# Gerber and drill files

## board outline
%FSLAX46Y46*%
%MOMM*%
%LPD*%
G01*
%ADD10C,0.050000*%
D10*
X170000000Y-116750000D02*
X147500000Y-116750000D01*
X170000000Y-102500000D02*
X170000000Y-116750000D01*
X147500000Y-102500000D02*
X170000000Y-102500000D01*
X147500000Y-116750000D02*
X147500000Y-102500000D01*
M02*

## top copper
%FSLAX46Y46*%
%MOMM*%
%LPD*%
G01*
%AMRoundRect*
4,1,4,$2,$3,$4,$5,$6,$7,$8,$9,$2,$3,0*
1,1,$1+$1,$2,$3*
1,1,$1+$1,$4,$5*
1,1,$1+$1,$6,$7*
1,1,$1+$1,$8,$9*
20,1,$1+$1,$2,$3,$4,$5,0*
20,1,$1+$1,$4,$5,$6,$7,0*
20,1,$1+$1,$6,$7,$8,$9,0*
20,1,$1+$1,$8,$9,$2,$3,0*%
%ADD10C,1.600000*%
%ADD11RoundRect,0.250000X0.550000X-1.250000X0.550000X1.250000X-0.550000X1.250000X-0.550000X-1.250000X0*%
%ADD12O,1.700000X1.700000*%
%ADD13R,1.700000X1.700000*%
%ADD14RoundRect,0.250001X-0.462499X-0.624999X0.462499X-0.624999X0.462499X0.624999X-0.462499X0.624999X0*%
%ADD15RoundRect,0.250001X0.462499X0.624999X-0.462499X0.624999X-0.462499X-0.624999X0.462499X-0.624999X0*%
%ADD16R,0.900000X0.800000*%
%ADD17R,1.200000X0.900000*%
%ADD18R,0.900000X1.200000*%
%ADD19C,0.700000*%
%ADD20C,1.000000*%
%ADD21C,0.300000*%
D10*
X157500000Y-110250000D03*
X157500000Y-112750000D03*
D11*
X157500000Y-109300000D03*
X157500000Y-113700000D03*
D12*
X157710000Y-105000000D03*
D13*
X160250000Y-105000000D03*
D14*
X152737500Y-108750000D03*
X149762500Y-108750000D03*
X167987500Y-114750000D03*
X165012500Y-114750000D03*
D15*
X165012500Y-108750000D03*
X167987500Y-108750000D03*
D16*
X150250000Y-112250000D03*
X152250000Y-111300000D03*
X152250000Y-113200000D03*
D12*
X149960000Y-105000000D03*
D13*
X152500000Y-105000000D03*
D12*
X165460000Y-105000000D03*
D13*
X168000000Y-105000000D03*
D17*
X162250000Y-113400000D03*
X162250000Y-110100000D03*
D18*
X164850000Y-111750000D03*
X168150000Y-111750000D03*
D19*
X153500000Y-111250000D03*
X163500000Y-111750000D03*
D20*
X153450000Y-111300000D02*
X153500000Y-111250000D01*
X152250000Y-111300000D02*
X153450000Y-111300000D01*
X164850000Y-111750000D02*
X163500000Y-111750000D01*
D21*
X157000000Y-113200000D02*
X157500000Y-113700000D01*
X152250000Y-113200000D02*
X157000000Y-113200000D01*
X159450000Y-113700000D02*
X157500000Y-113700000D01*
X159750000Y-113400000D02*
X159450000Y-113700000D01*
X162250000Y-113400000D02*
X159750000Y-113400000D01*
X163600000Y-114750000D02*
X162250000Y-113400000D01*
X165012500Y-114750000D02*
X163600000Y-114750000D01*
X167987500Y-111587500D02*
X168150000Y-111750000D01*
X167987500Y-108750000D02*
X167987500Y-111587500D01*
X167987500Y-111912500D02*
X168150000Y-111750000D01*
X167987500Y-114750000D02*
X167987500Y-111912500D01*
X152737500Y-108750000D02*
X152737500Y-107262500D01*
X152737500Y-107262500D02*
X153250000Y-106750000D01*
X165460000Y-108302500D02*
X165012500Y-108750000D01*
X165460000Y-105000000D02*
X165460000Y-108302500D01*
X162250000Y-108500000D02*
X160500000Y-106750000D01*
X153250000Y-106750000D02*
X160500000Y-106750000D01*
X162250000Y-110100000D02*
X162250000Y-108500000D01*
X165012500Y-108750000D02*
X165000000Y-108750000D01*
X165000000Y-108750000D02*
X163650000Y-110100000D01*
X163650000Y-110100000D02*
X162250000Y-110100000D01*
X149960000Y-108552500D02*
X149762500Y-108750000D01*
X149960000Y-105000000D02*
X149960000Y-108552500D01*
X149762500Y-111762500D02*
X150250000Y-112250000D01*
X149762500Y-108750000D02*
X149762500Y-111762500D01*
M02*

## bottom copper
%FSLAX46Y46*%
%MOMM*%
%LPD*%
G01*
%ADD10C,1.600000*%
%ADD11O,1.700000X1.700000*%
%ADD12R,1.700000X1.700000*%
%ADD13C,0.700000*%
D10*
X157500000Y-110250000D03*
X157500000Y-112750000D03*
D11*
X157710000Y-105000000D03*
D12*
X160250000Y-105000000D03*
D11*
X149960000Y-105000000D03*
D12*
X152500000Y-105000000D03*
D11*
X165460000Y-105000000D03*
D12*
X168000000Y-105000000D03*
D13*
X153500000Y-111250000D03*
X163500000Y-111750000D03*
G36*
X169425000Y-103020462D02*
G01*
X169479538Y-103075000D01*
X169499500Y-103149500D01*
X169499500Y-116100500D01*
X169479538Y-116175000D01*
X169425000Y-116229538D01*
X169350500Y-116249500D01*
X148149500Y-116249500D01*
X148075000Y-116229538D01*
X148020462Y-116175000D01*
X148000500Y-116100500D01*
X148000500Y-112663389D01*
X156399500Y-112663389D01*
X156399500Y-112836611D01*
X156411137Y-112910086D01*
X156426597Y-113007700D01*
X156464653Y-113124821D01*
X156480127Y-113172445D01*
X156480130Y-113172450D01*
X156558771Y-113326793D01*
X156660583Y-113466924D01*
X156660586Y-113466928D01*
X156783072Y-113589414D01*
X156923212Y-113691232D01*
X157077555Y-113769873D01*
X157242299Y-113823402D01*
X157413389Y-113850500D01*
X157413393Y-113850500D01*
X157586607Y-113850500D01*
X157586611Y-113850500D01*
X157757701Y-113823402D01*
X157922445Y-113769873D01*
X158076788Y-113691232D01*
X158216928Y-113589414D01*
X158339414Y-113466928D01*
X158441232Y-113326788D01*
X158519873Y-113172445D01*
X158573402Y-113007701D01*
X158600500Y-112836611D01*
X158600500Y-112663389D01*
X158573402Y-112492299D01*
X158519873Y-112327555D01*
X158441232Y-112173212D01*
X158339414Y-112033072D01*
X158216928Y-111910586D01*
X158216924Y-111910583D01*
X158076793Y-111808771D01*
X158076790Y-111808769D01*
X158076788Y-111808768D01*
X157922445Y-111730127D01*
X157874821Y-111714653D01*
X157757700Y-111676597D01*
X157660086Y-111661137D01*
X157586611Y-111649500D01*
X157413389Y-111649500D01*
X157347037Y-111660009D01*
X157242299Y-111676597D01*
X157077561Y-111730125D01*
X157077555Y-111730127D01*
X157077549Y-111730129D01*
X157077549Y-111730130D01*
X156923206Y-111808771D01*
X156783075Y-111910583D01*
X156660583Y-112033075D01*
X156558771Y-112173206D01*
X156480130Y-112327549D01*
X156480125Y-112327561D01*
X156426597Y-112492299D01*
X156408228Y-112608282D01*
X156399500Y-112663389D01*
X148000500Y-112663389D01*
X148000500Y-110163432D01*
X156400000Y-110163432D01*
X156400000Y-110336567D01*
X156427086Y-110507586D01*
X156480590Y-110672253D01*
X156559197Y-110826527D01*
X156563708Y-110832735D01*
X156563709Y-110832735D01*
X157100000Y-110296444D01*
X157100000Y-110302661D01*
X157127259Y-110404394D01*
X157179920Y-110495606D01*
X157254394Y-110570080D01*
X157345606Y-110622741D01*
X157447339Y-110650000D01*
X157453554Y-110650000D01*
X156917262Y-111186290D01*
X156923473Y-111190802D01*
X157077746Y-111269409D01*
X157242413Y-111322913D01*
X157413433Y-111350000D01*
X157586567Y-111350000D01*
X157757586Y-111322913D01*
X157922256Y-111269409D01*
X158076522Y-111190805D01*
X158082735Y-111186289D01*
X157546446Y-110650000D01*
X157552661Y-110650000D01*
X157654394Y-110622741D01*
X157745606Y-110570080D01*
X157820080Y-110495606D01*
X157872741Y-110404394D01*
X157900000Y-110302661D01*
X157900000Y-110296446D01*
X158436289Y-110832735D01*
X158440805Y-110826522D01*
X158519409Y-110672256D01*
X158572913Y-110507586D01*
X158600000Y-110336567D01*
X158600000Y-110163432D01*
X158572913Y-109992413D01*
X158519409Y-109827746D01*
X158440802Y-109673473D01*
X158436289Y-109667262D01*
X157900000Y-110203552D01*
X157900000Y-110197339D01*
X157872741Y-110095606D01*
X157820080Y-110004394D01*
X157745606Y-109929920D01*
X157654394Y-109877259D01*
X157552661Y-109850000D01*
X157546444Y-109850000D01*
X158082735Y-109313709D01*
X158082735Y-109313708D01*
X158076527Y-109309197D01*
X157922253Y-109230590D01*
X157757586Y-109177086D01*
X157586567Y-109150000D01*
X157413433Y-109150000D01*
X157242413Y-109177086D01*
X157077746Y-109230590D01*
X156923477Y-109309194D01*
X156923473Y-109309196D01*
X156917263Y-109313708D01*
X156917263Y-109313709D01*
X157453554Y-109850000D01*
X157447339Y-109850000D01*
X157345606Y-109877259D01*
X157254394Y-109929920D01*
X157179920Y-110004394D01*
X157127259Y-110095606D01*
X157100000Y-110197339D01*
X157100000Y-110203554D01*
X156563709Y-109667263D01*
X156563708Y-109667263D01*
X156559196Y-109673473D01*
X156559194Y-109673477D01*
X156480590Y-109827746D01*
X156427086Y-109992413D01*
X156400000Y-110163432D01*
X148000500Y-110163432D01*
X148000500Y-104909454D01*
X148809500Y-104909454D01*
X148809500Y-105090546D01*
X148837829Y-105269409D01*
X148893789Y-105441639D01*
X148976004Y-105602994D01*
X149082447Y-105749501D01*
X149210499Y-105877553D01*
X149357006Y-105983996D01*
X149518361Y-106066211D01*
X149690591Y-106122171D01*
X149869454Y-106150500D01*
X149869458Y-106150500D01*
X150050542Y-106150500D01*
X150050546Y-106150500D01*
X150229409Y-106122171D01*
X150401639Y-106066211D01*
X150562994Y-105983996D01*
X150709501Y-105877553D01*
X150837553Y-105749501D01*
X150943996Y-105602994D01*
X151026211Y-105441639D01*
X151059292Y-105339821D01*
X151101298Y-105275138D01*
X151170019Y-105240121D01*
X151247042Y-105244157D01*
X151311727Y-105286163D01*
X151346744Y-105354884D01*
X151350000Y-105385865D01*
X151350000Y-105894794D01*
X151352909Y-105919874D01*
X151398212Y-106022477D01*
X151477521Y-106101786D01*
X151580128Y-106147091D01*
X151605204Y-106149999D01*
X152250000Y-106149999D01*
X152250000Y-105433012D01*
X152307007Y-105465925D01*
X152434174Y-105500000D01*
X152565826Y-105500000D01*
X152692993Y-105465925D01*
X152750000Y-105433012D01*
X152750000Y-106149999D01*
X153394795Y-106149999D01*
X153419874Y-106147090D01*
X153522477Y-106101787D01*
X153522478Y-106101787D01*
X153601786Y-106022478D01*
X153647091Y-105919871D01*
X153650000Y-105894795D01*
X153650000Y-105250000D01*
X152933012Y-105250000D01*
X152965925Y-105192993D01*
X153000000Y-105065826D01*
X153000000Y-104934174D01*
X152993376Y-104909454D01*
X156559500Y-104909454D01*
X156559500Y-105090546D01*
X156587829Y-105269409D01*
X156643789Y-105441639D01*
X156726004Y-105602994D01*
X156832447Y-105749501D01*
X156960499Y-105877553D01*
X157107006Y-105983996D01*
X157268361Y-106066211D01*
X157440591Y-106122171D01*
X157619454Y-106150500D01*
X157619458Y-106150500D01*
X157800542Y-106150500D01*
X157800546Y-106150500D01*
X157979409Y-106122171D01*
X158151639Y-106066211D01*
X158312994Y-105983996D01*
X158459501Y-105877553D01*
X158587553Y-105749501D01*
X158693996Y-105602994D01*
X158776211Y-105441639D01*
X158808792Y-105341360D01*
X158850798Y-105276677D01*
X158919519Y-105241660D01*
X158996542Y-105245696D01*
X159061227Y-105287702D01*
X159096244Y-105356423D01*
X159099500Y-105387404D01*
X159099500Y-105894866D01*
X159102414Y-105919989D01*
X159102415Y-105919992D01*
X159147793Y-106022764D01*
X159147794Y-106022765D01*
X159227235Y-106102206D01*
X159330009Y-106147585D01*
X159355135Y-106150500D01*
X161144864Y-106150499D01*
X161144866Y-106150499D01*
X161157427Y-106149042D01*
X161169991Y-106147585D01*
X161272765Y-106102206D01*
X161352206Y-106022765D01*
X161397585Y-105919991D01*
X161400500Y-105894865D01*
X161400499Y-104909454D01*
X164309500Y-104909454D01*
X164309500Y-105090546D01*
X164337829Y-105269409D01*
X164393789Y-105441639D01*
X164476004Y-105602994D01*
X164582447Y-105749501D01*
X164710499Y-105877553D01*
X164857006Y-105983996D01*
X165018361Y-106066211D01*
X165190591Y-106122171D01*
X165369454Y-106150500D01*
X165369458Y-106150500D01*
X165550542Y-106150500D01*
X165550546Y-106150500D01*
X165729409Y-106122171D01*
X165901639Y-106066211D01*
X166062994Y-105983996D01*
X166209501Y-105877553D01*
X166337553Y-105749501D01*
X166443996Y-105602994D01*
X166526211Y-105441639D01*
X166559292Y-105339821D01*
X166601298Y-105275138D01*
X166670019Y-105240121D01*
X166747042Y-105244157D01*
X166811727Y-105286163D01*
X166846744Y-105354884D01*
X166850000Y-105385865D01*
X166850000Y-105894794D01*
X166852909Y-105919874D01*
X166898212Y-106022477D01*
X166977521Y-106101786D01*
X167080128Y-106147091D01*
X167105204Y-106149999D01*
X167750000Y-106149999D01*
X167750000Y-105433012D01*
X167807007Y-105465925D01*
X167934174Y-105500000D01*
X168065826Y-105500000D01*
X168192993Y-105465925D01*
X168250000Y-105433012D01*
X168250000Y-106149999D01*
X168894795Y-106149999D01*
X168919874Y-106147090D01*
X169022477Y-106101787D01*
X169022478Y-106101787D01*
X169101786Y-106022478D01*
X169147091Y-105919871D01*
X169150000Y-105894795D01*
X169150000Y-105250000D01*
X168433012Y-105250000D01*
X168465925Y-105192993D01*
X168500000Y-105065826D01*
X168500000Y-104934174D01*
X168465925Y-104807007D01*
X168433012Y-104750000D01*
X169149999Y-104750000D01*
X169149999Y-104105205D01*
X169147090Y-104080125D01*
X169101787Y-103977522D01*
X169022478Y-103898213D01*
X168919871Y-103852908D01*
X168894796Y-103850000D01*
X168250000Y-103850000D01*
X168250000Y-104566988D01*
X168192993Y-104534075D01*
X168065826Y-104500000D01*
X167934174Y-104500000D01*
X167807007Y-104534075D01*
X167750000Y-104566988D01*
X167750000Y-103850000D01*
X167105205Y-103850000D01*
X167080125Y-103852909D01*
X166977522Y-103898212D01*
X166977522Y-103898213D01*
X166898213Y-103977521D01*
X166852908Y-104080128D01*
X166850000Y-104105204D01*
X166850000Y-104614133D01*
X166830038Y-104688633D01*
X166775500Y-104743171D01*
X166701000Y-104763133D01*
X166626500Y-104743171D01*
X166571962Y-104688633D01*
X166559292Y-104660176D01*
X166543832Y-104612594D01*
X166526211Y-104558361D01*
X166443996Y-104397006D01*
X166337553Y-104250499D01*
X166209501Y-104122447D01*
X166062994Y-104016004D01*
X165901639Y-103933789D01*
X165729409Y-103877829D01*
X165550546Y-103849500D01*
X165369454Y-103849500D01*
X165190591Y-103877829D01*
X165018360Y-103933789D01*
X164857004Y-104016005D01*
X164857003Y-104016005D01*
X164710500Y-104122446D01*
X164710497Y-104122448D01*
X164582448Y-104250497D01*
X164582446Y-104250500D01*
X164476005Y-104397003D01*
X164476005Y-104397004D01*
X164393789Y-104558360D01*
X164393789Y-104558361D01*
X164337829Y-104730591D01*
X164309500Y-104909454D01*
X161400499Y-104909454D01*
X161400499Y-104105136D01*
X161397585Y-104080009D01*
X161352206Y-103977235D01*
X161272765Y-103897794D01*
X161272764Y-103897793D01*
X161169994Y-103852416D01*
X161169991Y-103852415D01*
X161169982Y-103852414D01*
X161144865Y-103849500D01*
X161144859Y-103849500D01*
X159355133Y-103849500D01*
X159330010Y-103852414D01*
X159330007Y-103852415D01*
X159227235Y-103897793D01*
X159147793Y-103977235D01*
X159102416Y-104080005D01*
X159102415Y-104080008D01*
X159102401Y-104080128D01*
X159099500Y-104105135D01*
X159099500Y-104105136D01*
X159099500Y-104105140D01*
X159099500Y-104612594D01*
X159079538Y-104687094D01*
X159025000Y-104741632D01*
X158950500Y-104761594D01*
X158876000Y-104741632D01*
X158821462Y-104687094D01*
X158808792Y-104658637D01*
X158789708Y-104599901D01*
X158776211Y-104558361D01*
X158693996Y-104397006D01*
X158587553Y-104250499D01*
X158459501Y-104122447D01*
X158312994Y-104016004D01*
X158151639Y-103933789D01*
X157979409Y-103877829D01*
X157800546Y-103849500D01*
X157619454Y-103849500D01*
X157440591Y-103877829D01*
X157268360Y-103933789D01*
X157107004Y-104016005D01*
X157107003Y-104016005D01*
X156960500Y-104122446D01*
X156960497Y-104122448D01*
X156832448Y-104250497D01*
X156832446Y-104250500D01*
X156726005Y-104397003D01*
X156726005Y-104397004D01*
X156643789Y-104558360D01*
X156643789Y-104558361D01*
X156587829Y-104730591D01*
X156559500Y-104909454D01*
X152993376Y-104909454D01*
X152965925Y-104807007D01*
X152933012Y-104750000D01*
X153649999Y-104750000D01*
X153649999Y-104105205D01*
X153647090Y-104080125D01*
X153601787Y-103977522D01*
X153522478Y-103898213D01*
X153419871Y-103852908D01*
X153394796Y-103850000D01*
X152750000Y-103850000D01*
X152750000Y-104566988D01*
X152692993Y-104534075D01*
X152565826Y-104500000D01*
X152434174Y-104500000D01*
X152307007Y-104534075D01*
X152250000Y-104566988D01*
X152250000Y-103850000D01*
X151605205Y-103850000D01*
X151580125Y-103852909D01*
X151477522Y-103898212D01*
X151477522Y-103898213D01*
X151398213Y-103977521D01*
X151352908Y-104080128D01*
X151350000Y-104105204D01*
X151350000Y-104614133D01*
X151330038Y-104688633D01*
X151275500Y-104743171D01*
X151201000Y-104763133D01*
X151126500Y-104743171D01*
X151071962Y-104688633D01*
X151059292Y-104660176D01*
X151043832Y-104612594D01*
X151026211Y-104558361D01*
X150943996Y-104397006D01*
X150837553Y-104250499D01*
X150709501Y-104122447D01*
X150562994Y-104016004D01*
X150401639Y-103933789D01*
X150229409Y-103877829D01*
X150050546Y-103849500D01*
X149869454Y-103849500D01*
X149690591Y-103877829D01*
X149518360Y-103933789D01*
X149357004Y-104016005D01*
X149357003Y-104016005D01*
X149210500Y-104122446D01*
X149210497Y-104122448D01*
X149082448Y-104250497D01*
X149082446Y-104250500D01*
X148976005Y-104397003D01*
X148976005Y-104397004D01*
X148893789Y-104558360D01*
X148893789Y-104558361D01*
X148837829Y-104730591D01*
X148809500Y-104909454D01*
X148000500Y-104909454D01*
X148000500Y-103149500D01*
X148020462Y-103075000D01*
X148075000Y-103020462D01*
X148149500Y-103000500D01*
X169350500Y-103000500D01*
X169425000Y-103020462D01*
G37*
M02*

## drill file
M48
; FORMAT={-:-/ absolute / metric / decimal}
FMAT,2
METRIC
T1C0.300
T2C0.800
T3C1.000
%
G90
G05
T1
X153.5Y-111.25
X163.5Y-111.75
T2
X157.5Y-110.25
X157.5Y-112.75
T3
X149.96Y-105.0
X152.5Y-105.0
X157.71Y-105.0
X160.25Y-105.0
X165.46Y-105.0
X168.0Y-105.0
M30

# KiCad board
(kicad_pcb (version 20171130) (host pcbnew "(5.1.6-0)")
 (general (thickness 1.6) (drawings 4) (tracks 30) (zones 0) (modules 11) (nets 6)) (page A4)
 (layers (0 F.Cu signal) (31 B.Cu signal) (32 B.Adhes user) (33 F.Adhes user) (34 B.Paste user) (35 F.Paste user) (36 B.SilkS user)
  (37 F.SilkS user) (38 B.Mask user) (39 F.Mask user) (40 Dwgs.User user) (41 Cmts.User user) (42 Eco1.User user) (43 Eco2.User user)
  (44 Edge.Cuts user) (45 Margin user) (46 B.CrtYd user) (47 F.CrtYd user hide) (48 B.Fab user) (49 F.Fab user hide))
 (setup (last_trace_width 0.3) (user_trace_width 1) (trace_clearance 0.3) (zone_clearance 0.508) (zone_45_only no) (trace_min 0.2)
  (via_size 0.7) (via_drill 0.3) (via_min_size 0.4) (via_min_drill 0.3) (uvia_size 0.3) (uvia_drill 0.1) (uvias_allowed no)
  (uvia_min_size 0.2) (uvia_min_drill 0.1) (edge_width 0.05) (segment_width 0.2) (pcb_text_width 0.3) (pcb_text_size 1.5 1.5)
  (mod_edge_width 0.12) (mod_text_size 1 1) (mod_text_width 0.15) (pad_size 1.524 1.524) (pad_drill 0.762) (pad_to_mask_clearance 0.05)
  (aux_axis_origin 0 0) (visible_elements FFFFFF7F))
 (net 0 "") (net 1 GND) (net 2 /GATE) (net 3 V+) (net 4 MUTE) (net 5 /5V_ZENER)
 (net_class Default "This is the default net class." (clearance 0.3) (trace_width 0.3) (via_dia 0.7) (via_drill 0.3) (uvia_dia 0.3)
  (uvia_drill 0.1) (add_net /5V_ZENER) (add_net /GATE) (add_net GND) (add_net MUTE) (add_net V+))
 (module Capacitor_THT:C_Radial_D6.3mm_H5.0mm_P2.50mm (layer F.Cu) (at 157.5 112.75 90)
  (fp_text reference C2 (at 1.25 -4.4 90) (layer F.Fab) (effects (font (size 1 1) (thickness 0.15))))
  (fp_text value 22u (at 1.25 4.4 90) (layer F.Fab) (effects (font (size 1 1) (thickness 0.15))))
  (pad 2 thru_hole circle (at 2.5 0 90) (size 1.6 1.6) (drill 0.8) (layers *.Cu *.Mask) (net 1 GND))
  (pad 1 thru_hole circle (at 0 0 90) (size 1.6 1.6) (drill 0.8) (layers *.Cu *.Mask) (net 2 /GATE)))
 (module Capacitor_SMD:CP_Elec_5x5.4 (layer F.Cu) (at 157.5 111.5 90)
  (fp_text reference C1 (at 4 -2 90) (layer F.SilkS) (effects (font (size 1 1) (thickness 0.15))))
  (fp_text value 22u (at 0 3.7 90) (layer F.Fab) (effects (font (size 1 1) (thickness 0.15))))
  (pad 2 smd roundrect (at 2.2 0 90) (size 3 1.6) (layers F.Cu F.Paste F.Mask) (roundrect_rratio 0.15625) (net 1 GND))
  (pad 1 smd roundrect (at -2.2 0 90) (size 3 1.6) (layers F.Cu F.Paste F.Mask) (roundrect_rratio 0.15625) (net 2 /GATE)))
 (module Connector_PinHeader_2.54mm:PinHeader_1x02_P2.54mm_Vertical (layer F.Cu) (at 160.25 105 270)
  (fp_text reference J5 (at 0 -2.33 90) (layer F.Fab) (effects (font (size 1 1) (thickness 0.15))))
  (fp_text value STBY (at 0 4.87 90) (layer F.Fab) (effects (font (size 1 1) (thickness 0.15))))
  (pad 2 thru_hole oval (at 0 2.54 270) (size 1.7 1.7) (drill 1) (layers *.Cu *.Mask))
  (pad 1 thru_hole rect (at 0 0 270) (size 1.7 1.7) (drill 1) (layers *.Cu *.Mask)))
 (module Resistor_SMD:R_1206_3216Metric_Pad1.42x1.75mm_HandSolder (layer F.Cu) (at 151.25 108.75)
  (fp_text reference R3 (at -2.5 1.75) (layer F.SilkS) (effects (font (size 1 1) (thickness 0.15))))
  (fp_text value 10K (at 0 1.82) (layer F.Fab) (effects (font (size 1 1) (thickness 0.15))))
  (pad 2 smd roundrect (at 1.4875 0) (size 1.425 1.75) (layers F.Cu F.Paste F.Mask) (roundrect_rratio 0.175439) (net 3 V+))
  (pad 1 smd roundrect (at -1.4875 0) (size 1.425 1.75) (layers F.Cu F.Paste F.Mask) (roundrect_rratio 0.175439) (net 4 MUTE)))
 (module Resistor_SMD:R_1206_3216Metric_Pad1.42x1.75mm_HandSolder (layer F.Cu) (at 166.5 114.75)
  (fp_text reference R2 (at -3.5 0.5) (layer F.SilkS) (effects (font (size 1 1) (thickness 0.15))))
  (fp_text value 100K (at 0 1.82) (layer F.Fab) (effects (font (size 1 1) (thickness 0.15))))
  (pad 2 smd roundrect (at 1.4875 0) (size 1.425 1.75) (layers F.Cu F.Paste F.Mask) (roundrect_rratio 0.175439) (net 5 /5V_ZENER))
  (pad 1 smd roundrect (at -1.4875 0) (size 1.425 1.75) (layers F.Cu F.Paste F.Mask) (roundrect_rratio 0.175439) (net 2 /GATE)))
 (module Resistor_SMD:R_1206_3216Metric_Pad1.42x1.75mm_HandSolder (layer F.Cu) (at 166.5 108.75 180)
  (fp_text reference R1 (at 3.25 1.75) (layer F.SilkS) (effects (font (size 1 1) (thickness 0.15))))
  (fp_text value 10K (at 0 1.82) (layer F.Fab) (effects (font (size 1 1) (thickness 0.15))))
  (pad 2 smd roundrect (at 1.4875 0 180) (size 1.425 1.75) (layers F.Cu F.Paste F.Mask) (roundrect_rratio 0.175439) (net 3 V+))
  (pad 1 smd roundrect (at -1.4875 0 180) (size 1.425 1.75) (layers F.Cu F.Paste F.Mask) (roundrect_rratio 0.175439) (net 5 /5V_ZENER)))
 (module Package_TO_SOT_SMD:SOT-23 (layer F.Cu) (at 151.25 112.25 180)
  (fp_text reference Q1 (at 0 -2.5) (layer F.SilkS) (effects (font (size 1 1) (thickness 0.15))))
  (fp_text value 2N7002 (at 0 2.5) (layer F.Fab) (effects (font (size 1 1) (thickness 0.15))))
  (pad 3 smd rect (at 1 0 180) (size 0.9 0.8) (layers F.Cu F.Paste F.Mask) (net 4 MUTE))
  (pad 2 smd rect (at -1 0.95 180) (size 0.9 0.8) (layers F.Cu F.Paste F.Mask) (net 1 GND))
  (pad 1 smd rect (at -1 -0.95 180) (size 0.9 0.8) (layers F.Cu F.Paste F.Mask) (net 2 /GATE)))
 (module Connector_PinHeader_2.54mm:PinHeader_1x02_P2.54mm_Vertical (layer F.Cu) (at 152.5 105 270)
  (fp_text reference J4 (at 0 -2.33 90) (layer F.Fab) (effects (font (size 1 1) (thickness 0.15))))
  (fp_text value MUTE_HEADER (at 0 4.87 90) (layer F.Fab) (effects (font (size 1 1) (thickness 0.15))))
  (pad 2 thru_hole oval (at 0 2.54 270) (size 1.7 1.7) (drill 1) (layers *.Cu *.Mask) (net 4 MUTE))
  (pad 1 thru_hole rect (at 0 0 270) (size 1.7 1.7) (drill 1) (layers *.Cu *.Mask) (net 1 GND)))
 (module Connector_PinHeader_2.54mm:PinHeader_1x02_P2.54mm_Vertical (layer F.Cu) (at 168 105 270)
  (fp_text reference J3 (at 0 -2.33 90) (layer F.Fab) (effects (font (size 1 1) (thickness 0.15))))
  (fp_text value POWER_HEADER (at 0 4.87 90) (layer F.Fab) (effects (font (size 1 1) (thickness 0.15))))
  (pad 2 thru_hole oval (at 0 2.54 270) (size 1.7 1.7) (drill 1) (layers *.Cu *.Mask) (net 3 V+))
  (pad 1 thru_hole rect (at 0 0 270) (size 1.7 1.7) (drill 1) (layers *.Cu *.Mask) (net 1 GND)))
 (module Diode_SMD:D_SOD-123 (layer F.Cu) (at 162.25 111.75 270)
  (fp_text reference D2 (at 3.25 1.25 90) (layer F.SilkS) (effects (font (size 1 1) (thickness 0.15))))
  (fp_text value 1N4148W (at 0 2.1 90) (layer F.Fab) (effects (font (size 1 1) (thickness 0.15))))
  (pad 2 smd rect (at 1.65 0 270) (size 0.9 1.2) (layers F.Cu F.Paste F.Mask) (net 2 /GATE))
  (pad 1 smd rect (at -1.65 0 270) (size 0.9 1.2) (layers F.Cu F.Paste F.Mask) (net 3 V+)))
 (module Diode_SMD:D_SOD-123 (layer F.Cu) (at 166.5 111.75 180)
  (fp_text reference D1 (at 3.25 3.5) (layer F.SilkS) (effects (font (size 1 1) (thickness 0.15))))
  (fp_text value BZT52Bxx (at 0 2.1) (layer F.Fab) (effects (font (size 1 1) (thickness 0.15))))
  (pad 2 smd rect (at 1.65 0 180) (size 0.9 1.2) (layers F.Cu F.Paste F.Mask) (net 1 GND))
  (pad 1 smd rect (at -1.65 0 180) (size 0.9 1.2) (layers F.Cu F.Paste F.Mask) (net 5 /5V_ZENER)))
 (gr_line (start 170 116.75) (end 147.5 116.75) (layer Edge.Cuts) (width 0.05))
 (gr_line (start 170 102.5) (end 170 116.75) (layer Edge.Cuts) (width 0.05))
 (gr_line (start 147.5 102.5) (end 170 102.5) (layer Edge.Cuts) (width 0.05))
 (gr_line (start 147.5 116.75) (end 147.5 102.5) (layer Edge.Cuts) (width 0.05))
 (via (at 153.5 111.25) (size 0.7) (drill 0.3) (layers F.Cu B.Cu) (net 1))
 (segment (start 153.45 111.3) (end 153.5 111.25) (width 1) (layer F.Cu) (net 1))
 (segment (start 152.25 111.3) (end 153.45 111.3) (width 1) (layer F.Cu) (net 1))
 (via (at 163.5 111.75) (size 0.7) (drill 0.3) (layers F.Cu B.Cu) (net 1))
 (segment (start 164.85 111.75) (end 163.5 111.75) (width 1) (layer F.Cu) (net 1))
 (segment (start 157 113.2) (end 157.5 113.7) (width 0.3) (layer F.Cu) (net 2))
 (segment (start 152.25 113.2) (end 157 113.2) (width 0.3) (layer F.Cu) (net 2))
 (segment (start 159.45 113.7) (end 157.5 113.7) (width 0.3) (layer F.Cu) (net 2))
 (segment (start 159.75 113.4) (end 159.45 113.7) (width 0.3) (layer F.Cu) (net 2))
 (segment (start 162.25 113.4) (end 159.75 113.4) (width 0.3) (layer F.Cu) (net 2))
 (segment (start 163.6 114.75) (end 162.25 113.4) (width 0.3) (layer F.Cu) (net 2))
 (segment (start 165.0125 114.75) (end 163.6 114.75) (width 0.3) (layer F.Cu) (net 2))
 (segment (start 167.9875 111.5875) (end 168.15 111.75) (width 0.3) (layer F.Cu) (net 5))
 (segment (start 167.9875 108.75) (end 167.9875 111.5875) (width 0.3) (layer F.Cu) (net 5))
 (segment (start 167.9875 111.9125) (end 168.15 111.75) (width 0.3) (layer F.Cu) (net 5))
 (segment (start 167.9875 114.75) (end 167.9875 111.9125) (width 0.3) (layer F.Cu) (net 5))
 (segment (start 152.7375 108.75) (end 152.7375 107.2625) (width 0.3) (layer F.Cu) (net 3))
 (segment (start 152.7375 107.2625) (end 153.25 106.75) (width 0.3) (layer F.Cu) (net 3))
 (segment (start 165.46 108.3025) (end 165.0125 108.75) (width 0.3) (layer F.Cu) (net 3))
 (segment (start 165.46 105) (end 165.46 108.3025) (width 0.3) (layer F.Cu) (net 3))
 (segment (start 162.25 108.5) (end 160.5 106.75) (width 0.3) (layer F.Cu) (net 3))
 (segment (start 153.25 106.75) (end 160.5 106.75) (width 0.3) (layer F.Cu) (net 3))
 (segment (start 162.25 110.1) (end 162.25 108.5) (width 0.3) (layer F.Cu) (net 3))
 (segment (start 165.0125 108.75) (end 165 108.75) (width 0.3) (layer F.Cu) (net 3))
 (segment (start 165 108.75) (end 163.65 110.1) (width 0.3) (layer F.Cu) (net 3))
 (segment (start 163.65 110.1) (end 162.25 110.1) (width 0.3) (layer F.Cu) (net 3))
 (segment (start 149.96 108.5525) (end 149.7625 108.75) (width 0.3) (layer F.Cu) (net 4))
 (segment (start 149.96 105) (end 149.96 108.5525) (width 0.3) (layer F.Cu) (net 4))
 (segment (start 149.7625 111.7625) (end 150.25 112.25) (width 0.3) (layer F.Cu) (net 4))
 (segment (start 149.7625 108.75) (end 149.7625 111.7625) (width 0.3) (layer F.Cu) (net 4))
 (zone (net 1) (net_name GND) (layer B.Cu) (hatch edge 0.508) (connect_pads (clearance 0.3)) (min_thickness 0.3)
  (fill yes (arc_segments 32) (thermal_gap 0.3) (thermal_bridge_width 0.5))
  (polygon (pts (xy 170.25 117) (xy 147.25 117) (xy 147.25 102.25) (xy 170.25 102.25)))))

